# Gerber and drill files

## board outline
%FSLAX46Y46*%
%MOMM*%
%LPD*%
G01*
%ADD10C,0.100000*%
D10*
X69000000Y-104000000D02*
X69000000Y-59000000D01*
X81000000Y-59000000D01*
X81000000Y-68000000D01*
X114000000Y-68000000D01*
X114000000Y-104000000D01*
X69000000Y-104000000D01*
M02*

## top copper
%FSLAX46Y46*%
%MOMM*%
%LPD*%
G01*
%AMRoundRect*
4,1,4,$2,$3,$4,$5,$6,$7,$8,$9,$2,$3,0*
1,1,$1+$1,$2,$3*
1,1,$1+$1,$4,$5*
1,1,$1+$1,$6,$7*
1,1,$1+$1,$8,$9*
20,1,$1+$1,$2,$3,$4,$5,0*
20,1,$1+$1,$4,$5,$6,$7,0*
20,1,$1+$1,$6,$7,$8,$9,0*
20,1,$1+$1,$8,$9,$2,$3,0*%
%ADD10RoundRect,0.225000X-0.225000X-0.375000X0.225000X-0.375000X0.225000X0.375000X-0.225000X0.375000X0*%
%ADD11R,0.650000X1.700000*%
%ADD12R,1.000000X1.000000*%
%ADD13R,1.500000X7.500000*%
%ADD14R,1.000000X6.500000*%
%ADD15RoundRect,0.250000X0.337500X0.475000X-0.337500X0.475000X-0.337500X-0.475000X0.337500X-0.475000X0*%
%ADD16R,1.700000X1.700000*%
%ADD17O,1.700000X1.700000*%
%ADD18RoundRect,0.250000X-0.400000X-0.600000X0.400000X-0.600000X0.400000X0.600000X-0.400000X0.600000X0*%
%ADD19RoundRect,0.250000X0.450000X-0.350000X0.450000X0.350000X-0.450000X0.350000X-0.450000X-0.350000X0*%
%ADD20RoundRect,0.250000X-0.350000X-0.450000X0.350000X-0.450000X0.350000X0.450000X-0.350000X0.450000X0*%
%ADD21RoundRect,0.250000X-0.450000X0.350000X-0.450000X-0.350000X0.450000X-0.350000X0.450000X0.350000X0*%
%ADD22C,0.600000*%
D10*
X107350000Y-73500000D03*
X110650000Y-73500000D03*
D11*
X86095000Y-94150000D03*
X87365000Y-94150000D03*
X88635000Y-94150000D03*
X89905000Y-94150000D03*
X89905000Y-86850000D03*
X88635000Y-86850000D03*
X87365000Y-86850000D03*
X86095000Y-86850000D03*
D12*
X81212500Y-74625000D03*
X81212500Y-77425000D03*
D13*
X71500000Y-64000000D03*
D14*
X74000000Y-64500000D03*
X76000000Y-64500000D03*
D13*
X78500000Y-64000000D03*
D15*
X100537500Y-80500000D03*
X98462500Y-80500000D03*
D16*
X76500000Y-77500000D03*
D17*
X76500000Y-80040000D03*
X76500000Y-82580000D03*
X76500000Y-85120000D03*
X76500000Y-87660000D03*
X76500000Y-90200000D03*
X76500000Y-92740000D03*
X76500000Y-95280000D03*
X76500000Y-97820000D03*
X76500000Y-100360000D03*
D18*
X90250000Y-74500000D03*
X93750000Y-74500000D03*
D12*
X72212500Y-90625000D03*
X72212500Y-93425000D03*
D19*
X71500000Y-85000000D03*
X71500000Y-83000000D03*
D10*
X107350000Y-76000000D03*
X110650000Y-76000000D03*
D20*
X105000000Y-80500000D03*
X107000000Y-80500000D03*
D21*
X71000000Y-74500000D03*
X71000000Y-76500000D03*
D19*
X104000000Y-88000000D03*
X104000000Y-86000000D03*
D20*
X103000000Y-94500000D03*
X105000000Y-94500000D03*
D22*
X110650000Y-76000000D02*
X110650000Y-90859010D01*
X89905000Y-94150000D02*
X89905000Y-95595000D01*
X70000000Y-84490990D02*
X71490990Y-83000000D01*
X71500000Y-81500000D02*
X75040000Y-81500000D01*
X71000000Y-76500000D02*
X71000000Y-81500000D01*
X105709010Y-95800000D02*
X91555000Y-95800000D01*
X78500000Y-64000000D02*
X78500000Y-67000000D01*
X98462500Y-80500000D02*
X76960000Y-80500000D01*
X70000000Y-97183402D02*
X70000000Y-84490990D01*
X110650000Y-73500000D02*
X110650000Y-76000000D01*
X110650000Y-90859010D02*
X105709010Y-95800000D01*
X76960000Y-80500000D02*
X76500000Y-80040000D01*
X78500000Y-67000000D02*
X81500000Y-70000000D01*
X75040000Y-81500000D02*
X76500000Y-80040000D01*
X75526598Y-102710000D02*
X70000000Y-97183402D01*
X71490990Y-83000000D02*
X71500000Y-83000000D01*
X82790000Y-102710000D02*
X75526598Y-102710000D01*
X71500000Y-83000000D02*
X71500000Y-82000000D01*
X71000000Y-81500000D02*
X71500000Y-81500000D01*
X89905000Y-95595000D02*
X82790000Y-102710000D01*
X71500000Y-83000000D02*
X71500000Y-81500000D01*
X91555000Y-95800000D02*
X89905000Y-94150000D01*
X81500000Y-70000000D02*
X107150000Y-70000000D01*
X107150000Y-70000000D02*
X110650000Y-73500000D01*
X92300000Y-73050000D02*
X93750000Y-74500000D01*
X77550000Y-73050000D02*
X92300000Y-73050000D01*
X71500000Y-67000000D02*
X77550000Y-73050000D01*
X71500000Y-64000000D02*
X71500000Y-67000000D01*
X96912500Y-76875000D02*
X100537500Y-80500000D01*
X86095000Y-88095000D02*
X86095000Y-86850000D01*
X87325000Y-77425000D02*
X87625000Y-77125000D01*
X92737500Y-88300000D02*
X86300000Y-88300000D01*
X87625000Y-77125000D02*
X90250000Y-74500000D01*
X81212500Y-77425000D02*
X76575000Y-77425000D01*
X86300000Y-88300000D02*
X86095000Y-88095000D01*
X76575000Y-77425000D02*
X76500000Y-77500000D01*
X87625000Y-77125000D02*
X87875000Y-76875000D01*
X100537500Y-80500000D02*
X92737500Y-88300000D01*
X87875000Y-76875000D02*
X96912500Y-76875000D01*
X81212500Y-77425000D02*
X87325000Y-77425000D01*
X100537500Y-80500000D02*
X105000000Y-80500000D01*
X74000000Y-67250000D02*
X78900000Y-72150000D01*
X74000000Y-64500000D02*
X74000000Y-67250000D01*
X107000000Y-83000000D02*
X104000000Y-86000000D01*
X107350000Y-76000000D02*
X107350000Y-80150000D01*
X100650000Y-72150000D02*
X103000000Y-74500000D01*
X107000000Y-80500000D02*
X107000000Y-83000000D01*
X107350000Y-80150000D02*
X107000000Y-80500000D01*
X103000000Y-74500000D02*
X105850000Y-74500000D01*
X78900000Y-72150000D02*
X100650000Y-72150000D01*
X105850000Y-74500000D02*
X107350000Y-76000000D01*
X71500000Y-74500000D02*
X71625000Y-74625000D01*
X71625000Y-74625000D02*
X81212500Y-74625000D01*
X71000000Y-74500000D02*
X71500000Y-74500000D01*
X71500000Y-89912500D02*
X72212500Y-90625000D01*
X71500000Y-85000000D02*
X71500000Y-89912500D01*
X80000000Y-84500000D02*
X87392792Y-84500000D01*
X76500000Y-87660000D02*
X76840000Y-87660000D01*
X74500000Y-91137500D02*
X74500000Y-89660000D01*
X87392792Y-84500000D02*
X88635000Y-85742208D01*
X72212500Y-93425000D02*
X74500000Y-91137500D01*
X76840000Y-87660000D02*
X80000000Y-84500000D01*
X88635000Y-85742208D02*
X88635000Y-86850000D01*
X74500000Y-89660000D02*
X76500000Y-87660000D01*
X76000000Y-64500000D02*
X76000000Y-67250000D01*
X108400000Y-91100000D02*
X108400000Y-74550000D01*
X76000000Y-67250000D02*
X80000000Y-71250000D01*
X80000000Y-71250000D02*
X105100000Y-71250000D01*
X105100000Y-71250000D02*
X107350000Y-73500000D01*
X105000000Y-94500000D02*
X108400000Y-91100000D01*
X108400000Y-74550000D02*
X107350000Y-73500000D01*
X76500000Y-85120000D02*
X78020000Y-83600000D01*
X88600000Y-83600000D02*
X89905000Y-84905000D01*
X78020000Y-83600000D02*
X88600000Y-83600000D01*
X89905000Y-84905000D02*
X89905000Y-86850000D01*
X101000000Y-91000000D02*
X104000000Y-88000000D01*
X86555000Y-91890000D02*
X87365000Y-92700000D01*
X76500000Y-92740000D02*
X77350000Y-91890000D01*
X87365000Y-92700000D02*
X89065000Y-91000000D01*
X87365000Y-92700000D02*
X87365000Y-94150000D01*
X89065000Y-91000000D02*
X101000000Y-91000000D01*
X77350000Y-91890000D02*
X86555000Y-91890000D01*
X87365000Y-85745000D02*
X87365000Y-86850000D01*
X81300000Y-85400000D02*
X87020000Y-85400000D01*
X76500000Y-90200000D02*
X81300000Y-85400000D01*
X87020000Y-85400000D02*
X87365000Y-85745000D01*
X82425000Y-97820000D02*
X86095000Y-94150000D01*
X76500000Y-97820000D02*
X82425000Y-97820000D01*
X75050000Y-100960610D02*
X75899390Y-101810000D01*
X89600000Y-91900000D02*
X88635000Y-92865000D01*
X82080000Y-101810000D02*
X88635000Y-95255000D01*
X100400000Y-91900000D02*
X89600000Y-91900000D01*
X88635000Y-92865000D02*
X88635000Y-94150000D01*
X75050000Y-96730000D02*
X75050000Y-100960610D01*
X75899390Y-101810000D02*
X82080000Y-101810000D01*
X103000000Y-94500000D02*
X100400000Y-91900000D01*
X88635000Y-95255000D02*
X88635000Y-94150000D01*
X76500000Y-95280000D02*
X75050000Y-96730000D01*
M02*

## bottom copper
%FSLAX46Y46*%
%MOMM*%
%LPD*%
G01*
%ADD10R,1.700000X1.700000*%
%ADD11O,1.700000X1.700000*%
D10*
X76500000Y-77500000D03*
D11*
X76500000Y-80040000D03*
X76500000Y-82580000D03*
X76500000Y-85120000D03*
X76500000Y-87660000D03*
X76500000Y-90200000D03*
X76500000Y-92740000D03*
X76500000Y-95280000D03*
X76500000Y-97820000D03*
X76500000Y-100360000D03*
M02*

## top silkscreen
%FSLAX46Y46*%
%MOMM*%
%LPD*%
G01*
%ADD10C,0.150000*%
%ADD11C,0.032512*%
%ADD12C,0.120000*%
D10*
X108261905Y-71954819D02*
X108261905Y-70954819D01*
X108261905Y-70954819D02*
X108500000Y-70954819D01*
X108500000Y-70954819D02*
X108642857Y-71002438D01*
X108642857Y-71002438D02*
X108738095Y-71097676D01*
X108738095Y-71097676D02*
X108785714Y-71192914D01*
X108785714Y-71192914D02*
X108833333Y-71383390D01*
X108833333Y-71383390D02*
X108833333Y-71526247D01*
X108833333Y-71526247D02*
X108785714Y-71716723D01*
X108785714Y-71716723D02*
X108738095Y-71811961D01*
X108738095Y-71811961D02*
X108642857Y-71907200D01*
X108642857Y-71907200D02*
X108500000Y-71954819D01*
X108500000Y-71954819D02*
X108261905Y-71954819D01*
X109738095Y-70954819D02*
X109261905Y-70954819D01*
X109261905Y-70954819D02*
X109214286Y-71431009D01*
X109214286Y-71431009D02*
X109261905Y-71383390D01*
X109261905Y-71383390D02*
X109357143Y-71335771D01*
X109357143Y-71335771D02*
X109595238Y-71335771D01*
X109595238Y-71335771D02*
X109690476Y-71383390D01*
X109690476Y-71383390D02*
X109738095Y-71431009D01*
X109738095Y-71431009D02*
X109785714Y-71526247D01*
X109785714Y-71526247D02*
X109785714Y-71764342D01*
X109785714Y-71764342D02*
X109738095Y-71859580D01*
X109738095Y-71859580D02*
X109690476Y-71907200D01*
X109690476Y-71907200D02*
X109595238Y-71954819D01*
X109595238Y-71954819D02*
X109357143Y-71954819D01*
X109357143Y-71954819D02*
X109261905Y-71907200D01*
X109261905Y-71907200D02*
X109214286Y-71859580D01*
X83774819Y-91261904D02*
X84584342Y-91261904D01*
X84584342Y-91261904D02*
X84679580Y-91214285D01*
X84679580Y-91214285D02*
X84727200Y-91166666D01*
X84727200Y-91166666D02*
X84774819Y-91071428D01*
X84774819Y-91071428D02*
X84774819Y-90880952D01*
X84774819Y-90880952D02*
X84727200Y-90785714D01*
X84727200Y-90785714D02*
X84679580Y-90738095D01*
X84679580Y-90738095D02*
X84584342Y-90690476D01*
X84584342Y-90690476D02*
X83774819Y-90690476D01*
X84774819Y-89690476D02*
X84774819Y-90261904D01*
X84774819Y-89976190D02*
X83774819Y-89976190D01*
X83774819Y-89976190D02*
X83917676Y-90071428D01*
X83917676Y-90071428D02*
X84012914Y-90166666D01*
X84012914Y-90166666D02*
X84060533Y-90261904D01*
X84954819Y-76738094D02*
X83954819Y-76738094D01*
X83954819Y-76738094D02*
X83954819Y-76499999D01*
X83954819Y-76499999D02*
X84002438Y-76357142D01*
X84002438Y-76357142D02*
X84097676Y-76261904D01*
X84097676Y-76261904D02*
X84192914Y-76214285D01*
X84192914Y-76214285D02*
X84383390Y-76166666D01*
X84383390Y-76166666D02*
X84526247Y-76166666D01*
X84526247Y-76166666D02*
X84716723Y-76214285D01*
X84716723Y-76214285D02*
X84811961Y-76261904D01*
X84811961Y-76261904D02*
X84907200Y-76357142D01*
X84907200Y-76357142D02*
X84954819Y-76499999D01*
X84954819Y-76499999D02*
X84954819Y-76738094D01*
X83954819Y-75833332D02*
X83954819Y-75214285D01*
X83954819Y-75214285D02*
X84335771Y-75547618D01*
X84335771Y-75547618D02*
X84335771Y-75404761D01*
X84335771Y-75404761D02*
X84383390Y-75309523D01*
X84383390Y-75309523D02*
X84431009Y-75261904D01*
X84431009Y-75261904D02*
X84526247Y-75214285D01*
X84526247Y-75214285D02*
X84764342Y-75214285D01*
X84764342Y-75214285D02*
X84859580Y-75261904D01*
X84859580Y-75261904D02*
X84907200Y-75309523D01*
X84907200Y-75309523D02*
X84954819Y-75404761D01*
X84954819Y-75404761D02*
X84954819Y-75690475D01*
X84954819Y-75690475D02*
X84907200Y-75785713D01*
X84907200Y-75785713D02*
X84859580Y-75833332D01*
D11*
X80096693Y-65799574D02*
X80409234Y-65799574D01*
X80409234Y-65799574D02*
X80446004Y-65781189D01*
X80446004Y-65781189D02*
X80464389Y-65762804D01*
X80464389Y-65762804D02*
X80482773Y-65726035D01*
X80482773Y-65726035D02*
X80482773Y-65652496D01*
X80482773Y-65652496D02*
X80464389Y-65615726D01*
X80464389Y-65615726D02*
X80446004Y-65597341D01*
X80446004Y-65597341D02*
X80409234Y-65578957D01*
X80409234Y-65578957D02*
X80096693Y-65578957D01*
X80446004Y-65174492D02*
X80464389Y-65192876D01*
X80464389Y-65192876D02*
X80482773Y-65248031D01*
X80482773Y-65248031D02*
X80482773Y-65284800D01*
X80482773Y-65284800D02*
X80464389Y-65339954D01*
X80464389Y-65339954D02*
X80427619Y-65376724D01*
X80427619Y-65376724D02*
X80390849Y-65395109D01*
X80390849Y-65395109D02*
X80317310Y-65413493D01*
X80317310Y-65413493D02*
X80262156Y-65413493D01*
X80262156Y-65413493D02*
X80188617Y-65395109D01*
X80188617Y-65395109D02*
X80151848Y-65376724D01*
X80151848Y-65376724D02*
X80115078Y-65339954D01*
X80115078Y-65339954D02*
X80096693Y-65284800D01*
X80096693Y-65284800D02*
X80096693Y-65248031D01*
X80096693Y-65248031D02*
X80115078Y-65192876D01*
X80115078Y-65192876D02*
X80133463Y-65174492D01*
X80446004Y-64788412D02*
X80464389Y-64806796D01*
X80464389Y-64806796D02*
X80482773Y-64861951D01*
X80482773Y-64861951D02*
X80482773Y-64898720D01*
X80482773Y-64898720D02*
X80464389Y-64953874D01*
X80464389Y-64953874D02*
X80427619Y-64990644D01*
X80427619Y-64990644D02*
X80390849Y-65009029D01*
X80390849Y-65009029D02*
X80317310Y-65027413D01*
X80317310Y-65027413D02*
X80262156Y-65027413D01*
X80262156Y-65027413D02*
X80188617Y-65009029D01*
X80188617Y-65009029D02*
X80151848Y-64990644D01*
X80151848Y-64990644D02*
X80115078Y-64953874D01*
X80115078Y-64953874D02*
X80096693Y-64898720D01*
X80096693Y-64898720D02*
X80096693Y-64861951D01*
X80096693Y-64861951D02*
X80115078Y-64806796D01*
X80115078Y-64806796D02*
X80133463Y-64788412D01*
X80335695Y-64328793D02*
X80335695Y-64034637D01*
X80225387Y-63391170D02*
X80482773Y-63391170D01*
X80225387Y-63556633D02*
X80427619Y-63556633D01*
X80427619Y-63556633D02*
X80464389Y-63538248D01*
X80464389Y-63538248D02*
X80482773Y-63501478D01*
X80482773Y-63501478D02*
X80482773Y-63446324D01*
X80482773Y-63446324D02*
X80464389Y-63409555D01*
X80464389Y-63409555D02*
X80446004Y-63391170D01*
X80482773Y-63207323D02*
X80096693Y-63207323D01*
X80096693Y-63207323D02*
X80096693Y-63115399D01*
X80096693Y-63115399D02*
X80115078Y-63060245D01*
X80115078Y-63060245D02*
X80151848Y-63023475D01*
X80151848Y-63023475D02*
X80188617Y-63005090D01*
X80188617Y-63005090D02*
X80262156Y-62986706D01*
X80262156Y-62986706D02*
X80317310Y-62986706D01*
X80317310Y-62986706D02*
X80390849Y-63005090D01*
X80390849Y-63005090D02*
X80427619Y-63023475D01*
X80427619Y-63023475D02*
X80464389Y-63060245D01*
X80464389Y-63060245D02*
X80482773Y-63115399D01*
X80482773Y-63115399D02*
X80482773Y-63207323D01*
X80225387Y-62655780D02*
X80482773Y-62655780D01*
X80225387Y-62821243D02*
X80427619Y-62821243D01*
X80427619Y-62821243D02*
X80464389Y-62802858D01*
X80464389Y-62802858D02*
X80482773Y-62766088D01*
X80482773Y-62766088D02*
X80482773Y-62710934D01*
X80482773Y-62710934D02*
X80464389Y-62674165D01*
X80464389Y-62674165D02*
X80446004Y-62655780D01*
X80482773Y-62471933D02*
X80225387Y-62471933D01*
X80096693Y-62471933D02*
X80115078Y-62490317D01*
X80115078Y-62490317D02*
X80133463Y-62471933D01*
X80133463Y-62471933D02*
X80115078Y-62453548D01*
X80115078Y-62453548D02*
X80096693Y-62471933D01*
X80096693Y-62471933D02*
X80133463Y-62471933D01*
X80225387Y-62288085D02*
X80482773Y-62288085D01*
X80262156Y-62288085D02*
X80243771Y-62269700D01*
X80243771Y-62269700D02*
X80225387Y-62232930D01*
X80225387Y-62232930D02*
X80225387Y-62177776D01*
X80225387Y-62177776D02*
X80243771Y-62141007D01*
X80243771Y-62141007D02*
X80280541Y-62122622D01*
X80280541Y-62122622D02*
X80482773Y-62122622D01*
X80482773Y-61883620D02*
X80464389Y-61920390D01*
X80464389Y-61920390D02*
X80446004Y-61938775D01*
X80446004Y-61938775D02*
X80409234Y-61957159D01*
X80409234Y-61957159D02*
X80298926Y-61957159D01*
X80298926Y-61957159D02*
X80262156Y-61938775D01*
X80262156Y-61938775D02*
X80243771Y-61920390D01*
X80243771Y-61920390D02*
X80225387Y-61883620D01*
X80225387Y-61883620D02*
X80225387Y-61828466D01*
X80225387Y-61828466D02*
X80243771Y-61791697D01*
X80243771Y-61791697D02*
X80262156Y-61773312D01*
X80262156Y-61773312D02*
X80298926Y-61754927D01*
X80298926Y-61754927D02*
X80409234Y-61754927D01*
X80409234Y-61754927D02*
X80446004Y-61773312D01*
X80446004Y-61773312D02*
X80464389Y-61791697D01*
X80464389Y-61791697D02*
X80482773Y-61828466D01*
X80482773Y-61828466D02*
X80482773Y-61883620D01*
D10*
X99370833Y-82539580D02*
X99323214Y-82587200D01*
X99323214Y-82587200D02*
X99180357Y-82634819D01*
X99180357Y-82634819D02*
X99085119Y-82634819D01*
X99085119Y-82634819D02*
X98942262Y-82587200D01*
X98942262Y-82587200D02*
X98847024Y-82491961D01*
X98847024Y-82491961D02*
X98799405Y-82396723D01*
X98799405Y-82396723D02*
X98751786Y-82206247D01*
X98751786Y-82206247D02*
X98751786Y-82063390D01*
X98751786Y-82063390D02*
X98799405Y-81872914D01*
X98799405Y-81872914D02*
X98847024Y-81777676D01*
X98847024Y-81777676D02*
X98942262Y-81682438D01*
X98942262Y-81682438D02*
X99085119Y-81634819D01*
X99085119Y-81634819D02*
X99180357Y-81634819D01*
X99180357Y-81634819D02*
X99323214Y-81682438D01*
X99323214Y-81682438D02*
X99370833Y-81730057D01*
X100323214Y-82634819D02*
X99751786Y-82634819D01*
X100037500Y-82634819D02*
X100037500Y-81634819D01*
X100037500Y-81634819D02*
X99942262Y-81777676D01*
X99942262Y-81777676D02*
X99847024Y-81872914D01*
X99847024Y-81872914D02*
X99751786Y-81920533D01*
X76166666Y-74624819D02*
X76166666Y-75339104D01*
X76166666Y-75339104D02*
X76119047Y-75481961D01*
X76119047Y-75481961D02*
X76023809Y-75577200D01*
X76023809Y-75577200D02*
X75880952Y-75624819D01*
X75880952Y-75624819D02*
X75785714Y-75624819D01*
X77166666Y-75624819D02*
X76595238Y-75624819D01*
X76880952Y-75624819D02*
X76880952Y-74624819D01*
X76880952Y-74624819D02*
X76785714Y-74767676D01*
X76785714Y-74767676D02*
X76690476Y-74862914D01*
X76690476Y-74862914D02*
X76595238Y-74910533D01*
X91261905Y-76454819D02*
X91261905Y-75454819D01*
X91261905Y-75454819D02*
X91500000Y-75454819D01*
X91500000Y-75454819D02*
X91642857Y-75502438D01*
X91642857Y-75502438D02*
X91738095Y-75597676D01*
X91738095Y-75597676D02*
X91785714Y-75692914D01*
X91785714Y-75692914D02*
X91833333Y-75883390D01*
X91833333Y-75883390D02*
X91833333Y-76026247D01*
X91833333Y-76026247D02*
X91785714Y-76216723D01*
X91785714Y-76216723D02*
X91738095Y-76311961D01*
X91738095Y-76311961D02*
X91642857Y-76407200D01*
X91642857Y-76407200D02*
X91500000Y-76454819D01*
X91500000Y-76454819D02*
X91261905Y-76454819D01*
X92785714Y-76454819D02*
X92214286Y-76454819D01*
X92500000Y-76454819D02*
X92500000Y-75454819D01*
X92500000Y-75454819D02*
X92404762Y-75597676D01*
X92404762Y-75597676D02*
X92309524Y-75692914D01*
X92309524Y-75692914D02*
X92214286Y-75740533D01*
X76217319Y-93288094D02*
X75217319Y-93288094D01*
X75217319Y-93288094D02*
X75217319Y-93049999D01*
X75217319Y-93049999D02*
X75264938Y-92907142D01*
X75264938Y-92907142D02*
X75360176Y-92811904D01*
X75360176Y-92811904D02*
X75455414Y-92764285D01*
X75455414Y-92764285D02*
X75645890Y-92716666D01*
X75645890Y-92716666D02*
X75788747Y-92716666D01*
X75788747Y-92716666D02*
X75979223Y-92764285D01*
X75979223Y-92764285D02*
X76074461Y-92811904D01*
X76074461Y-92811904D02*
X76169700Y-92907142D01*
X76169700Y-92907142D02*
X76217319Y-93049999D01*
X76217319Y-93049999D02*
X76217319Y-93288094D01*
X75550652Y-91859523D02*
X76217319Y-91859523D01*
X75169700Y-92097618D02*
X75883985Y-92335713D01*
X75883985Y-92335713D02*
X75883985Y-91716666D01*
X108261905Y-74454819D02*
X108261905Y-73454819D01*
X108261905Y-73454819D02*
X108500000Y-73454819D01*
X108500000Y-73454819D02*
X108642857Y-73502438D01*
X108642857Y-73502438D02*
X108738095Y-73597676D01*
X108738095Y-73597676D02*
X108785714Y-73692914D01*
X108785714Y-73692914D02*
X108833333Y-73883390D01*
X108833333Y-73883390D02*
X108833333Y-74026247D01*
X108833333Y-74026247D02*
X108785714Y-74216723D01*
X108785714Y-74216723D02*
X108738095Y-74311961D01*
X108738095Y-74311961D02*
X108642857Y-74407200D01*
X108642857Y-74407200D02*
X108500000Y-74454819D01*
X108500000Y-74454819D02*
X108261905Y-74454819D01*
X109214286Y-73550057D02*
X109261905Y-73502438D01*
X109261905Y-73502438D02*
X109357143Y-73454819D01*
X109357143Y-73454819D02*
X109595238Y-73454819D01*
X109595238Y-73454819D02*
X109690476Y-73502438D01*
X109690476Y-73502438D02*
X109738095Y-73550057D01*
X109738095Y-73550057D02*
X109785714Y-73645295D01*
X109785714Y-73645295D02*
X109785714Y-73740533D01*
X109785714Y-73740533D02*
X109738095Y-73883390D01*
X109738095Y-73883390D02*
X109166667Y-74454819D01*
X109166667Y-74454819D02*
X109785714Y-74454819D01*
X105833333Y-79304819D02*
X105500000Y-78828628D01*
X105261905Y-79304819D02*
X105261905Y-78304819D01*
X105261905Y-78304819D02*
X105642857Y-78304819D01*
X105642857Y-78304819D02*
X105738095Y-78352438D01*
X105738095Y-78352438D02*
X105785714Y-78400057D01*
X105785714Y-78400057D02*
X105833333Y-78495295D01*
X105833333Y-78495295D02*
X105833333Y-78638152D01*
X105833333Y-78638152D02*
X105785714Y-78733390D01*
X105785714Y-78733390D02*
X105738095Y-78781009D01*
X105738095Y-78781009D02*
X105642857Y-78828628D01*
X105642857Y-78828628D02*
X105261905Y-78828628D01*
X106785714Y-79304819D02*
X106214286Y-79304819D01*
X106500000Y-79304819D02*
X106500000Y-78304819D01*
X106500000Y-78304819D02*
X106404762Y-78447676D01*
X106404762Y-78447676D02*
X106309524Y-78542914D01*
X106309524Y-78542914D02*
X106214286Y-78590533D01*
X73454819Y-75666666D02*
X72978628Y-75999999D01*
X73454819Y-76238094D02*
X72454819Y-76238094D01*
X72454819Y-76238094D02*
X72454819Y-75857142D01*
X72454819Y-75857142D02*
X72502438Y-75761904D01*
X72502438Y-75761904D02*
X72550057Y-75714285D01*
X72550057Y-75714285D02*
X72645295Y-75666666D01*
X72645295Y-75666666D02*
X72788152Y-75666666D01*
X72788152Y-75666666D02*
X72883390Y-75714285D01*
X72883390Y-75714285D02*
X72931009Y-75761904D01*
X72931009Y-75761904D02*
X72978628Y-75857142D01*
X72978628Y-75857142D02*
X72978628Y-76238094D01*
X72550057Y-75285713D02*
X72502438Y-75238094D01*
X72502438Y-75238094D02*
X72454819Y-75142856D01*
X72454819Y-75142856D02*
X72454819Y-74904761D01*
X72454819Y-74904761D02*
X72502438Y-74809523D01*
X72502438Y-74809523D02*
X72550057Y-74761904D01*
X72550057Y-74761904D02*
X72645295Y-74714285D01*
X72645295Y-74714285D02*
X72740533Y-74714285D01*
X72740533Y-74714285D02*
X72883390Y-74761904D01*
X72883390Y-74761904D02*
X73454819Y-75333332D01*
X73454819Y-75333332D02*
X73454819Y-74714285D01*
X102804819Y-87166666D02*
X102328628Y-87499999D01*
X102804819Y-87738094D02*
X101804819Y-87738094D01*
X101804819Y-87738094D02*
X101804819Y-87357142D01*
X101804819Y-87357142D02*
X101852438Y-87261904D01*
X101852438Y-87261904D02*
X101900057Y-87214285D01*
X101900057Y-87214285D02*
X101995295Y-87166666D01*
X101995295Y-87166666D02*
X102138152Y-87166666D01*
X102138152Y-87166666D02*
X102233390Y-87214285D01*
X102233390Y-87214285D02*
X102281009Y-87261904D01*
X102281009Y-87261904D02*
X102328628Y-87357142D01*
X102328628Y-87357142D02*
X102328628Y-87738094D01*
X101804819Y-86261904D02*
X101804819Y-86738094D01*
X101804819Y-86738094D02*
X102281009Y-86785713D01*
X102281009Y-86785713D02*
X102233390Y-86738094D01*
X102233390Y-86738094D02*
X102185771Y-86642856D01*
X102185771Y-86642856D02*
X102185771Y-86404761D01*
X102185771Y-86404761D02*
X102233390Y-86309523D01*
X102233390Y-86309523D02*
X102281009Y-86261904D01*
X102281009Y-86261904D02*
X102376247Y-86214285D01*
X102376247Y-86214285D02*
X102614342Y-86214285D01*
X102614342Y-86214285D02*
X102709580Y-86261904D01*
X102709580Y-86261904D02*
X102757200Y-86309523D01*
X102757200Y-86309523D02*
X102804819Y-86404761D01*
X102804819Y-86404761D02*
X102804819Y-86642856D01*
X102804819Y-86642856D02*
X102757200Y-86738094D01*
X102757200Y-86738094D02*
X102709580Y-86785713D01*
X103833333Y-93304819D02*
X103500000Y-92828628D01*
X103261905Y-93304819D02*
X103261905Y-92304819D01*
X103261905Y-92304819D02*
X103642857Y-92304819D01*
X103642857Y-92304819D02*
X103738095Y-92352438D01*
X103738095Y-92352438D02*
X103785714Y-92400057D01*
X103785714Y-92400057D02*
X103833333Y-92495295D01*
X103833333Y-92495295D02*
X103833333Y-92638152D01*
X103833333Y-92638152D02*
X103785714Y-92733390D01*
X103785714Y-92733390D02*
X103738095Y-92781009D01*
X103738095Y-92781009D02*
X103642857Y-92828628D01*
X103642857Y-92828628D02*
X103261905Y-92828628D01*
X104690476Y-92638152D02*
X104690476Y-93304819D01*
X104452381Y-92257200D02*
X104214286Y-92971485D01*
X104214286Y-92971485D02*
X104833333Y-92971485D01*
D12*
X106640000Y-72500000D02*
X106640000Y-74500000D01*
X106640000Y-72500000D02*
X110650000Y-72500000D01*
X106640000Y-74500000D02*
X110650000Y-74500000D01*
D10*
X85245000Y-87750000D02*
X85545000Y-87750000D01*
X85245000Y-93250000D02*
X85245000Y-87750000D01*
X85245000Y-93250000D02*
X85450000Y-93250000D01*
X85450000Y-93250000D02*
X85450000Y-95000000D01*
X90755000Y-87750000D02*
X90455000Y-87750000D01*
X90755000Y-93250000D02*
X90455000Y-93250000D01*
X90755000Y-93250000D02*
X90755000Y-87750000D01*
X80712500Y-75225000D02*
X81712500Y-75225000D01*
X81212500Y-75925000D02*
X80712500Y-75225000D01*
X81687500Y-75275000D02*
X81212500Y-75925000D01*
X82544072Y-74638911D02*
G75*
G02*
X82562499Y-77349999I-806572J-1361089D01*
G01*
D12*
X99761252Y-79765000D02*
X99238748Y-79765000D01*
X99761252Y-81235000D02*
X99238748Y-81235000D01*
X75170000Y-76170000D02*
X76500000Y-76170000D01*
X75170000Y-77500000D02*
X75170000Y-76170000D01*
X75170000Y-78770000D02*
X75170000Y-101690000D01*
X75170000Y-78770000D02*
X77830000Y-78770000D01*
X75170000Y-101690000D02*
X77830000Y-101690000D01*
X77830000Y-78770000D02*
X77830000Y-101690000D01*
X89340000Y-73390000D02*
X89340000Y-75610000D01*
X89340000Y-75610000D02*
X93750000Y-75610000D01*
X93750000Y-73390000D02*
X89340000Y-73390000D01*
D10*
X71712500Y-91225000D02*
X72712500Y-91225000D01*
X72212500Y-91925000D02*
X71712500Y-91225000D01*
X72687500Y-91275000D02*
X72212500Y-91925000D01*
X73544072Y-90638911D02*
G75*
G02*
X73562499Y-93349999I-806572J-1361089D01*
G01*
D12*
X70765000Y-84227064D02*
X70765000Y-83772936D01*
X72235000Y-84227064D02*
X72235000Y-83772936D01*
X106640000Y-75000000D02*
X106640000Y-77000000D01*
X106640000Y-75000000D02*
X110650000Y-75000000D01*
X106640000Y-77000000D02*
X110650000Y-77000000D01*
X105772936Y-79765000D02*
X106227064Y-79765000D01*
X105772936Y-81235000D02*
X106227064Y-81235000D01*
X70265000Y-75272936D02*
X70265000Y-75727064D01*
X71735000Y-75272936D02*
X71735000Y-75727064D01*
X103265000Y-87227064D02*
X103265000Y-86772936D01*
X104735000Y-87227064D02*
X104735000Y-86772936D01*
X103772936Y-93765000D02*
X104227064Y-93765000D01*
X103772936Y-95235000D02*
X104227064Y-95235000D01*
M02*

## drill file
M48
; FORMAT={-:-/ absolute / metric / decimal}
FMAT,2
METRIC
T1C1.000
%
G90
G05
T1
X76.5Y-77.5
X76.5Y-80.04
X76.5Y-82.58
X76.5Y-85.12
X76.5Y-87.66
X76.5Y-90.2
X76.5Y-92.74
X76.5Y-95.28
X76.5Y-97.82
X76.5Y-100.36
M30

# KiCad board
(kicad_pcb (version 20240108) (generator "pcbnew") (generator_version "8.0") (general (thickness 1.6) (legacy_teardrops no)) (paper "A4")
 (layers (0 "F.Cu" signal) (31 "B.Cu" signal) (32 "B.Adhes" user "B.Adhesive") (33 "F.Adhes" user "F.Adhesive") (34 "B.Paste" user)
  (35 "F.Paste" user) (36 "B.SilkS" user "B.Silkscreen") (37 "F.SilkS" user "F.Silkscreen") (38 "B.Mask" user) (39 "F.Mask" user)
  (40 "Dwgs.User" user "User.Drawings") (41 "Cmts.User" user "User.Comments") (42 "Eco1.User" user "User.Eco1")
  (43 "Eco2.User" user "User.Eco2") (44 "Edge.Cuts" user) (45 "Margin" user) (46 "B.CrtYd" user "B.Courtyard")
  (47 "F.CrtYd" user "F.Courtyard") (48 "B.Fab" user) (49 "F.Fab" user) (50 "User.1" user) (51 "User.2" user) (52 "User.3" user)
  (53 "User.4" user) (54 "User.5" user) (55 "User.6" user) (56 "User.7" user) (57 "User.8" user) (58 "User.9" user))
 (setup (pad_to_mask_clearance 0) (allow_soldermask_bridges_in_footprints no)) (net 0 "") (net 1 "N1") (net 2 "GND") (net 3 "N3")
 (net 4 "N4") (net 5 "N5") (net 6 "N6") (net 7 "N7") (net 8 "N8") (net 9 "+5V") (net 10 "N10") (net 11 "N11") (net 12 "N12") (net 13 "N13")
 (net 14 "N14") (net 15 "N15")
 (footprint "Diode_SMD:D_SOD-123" (layer "F.Cu") (at 109 73.5)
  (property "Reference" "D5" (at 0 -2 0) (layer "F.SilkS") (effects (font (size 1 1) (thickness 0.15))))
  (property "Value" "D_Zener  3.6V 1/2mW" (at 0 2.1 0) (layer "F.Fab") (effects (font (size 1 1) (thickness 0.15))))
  (fp_line (start -2.36 -1) (end -2.36 1) (stroke (width 0.12) (type solid)) (layer "F.SilkS"))
  (fp_line (start -2.36 -1) (end 1.65 -1) (stroke (width 0.12) (type solid)) (layer "F.SilkS"))
  (fp_line (start -2.36 1) (end 1.65 1) (stroke (width 0.12) (type solid)) (layer "F.SilkS"))
  (pad "1" smd roundrect (at -1.65 0) (size 0.9 1.2) (layers "F.Cu" "F.Paste" "F.Mask") (roundrect_rratio 0.25) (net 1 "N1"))
  (pad "2" smd roundrect (at 1.65 0) (size 0.9 1.2) (layers "F.Cu" "F.Paste" "F.Mask") (roundrect_rratio 0.25) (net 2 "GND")))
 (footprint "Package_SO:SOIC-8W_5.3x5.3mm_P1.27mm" (layer "F.Cu") (at 88 90.5 90)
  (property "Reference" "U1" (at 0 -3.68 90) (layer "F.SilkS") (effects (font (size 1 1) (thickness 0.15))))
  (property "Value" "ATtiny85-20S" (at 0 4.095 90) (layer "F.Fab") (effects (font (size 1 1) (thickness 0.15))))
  (fp_line (start 2.75 -2.755) (end 2.75 -2.455) (stroke (width 0.15) (type solid)) (layer "F.SilkS"))
  (fp_line (start -2.75 -2.755) (end 2.75 -2.755) (stroke (width 0.15) (type solid)) (layer "F.SilkS"))
  (fp_line (start -2.75 -2.755) (end -2.75 -2.55) (stroke (width 0.15) (type solid)) (layer "F.SilkS"))
  (fp_line (start -2.75 -2.55) (end -4.5 -2.55) (stroke (width 0.15) (type solid)) (layer "F.SilkS"))
  (fp_line (start 2.75 2.755) (end 2.75 2.455) (stroke (width 0.15) (type solid)) (layer "F.SilkS"))
  (fp_line (start -2.75 2.755) (end -2.75 2.455) (stroke (width 0.15) (type solid)) (layer "F.SilkS"))
  (fp_line (start -2.75 2.755) (end 2.75 2.755) (stroke (width 0.15) (type solid)) (layer "F.SilkS"))
  (pad "1" smd rect (at -3.65 -1.905 90) (size 1.7 0.65) (layers "F.Cu" "F.Paste" "F.Mask") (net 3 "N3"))
  (pad "2" smd rect (at -3.65 -0.635 90) (size 1.7 0.65) (layers "F.Cu" "F.Paste" "F.Mask") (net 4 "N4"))
  (pad "3" smd rect (at -3.65 0.635 90) (size 1.7 0.65) (layers "F.Cu" "F.Paste" "F.Mask") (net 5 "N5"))
  (pad "4" smd rect (at -3.65 1.905 90) (size 1.7 0.65) (layers "F.Cu" "F.Paste" "F.Mask") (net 2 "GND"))
  (pad "5" smd rect (at 3.65 1.905 90) (size 1.7 0.65) (layers "F.Cu" "F.Paste" "F.Mask") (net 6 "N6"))
  (pad "6" smd rect (at 3.65 0.635 90) (size 1.7 0.65) (layers "F.Cu" "F.Paste" "F.Mask") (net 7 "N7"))
  (pad "7" smd rect (at 3.65 -0.635 90) (size 1.7 0.65) (layers "F.Cu" "F.Paste" "F.Mask") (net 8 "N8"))
  (pad "8" smd rect (at 3.65 -1.905 90) (size 1.7 0.65) (layers "F.Cu" "F.Paste" "F.Mask") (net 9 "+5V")))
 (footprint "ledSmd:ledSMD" (layer "F.Cu") (at 81.2125 76.425 -90)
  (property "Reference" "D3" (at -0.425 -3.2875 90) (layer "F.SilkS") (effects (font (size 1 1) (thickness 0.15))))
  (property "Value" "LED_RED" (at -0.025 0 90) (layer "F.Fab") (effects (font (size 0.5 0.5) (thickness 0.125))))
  (fp_line (start -1.2 0.5) (end -1.2 -0.5) (stroke (width 0.15) (type solid)) (layer "F.SilkS"))
  (fp_line (start -0.5 0) (end -1.2 0.5) (stroke (width 0.15) (type solid)) (layer "F.SilkS"))
  (fp_line (start -1.15 -0.475) (end -0.5 0) (stroke (width 0.15) (type solid)) (layer "F.SilkS"))
  (fp_arc (start -1.786089 -1.331572) (mid -0.435753 -2.107089) (end 0.924999 -1.349999) (stroke (width 0.15) (type solid))
   (layer "F.SilkS"))
  (pad "1" smd rect (at -1.8 0 270) (size 1 1) (layers "F.Cu" "F.Paste" "F.Mask") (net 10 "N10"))
  (pad "2" smd rect (at 1 0 270) (size 1 1) (layers "F.Cu" "F.Paste" "F.Mask") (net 9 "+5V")))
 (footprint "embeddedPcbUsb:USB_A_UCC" (layer "F.Cu") (at 75 64.2 -90)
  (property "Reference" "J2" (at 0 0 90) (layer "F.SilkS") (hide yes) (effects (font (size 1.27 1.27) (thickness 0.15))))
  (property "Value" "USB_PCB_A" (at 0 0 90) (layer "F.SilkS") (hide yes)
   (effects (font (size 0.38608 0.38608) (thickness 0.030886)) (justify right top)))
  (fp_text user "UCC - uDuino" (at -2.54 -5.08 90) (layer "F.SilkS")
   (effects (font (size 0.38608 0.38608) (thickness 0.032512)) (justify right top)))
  (pad "1" smd rect (at -0.2 3.5 270) (size 7.5 1.5) (layers "F.Cu" "F.Paste" "F.Mask") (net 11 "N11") (solder_mask_margin 0.1016))
  (pad "2" smd rect (at 0.3 1 270) (size 6.5 1) (layers "F.Cu" "F.Paste" "F.Mask") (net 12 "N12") (solder_mask_margin 0.1016))
  (pad "3" smd rect (at 0.3 -1 270) (size 6.5 1) (layers "F.Cu" "F.Paste" "F.Mask") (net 1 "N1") (solder_mask_margin 0.1016))
  (pad "4" smd rect (at -0.2 -3.5 270) (size 7.5 1.5) (layers "F.Cu" "F.Paste" "F.Mask") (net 2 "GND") (solder_mask_margin 0.1016)))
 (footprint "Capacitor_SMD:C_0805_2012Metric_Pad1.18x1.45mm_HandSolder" (layer "F.Cu") (at 99.5 80.5 180)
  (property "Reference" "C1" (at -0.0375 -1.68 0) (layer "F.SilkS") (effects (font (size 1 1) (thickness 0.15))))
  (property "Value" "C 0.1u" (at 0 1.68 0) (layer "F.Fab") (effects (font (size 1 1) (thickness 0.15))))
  (fp_line (start -0.261252 0.735) (end 0.261252 0.735) (stroke (width 0.12) (type solid)) (layer "F.SilkS"))
  (fp_line (start -0.261252 -0.735) (end 0.261252 -0.735) (stroke (width 0.12) (type solid)) (layer "F.SilkS"))
  (pad "1" smd roundrect (at -1.0375 0 180) (size 1.175 1.45) (layers "F.Cu" "F.Paste" "F.Mask") (roundrect_rratio 0.212766) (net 9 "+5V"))
  (pad "2" smd roundrect (at 1.0375 0 180) (size 1.175 1.45) (layers "F.Cu" "F.Paste" "F.Mask") (roundrect_rratio 0.212766) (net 2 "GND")))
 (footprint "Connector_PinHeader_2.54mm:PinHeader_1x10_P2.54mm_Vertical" (layer "F.Cu") (at 76.5 77.5)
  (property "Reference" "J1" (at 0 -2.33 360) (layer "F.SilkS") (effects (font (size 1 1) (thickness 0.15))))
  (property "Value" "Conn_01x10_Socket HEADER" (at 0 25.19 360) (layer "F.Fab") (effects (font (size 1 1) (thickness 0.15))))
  (fp_line (start -1.33 -1.33) (end 0 -1.33) (stroke (width 0.12) (type solid)) (layer "F.SilkS"))
  (fp_line (start -1.33 0) (end -1.33 -1.33) (stroke (width 0.12) (type solid)) (layer "F.SilkS"))
  (fp_line (start -1.33 1.27) (end -1.33 24.19) (stroke (width 0.12) (type solid)) (layer "F.SilkS"))
  (fp_line (start -1.33 1.27) (end 1.33 1.27) (stroke (width 0.12) (type solid)) (layer "F.SilkS"))
  (fp_line (start -1.33 24.19) (end 1.33 24.19) (stroke (width 0.12) (type solid)) (layer "F.SilkS"))
  (fp_line (start 1.33 1.27) (end 1.33 24.19) (stroke (width 0.12) (type solid)) (layer "F.SilkS"))
  (pad "1" thru_hole rect (at 0 0) (size 1.7 1.7) (drill 1) (layers "*.Cu" "*.Mask") (remove_unused_layers no) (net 9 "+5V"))
  (pad "2" thru_hole oval (at 0 2.54) (size 1.7 1.7) (drill 1) (layers "*.Cu" "*.Mask") (remove_unused_layers no) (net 2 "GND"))
  (pad "3" thru_hole oval (at 0 5.08) (size 1.7 1.7) (drill 1) (layers "*.Cu" "*.Mask") (remove_unused_layers no) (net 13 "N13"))
  (pad "4" thru_hole oval (at 0 7.62) (size 1.7 1.7) (drill 1) (layers "*.Cu" "*.Mask") (remove_unused_layers no) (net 6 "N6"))
  (pad "5" thru_hole oval (at 0 10.16) (size 1.7 1.7) (drill 1) (layers "*.Cu" "*.Mask") (remove_unused_layers no) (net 7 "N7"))
  (pad "6" thru_hole oval (at 0 12.7) (size 1.7 1.7) (drill 1) (layers "*.Cu" "*.Mask") (remove_unused_layers no) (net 8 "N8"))
  (pad "7" thru_hole oval (at 0 15.24) (size 1.7 1.7) (drill 1) (layers "*.Cu" "*.Mask") (remove_unused_layers no) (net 4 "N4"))
  (pad "8" thru_hole oval (at 0 17.78) (size 1.7 1.7) (drill 1) (layers "*.Cu" "*.Mask") (remove_unused_layers no) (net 5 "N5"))
  (pad "9" thru_hole oval (at 0 20.32) (size 1.7 1.7) (drill 1) (layers "*.Cu" "*.Mask") (remove_unused_layers no) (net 3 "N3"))
  (pad "10" thru_hole oval (at 0 22.86) (size 1.7 1.7) (drill 1) (layers "*.Cu" "*.Mask") (remove_unused_layers no) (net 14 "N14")))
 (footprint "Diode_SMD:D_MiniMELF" (layer "F.Cu") (at 92 74.5)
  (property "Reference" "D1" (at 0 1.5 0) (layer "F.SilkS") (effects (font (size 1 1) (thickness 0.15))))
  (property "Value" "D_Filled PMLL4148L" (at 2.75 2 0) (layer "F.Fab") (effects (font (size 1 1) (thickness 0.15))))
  (fp_line (start -2.66 -1.11) (end -2.66 1.11) (stroke (width 0.12) (type solid)) (layer "F.SilkS"))
  (fp_line (start -2.66 1.11) (end 1.75 1.11) (stroke (width 0.12) (type solid)) (layer "F.SilkS"))
  (fp_line (start 1.75 -1.11) (end -2.66 -1.11) (stroke (width 0.12) (type solid)) (layer "F.SilkS"))
  (pad "1" smd roundrect (at -1.75 0) (size 1.3 1.7) (layers "F.Cu" "F.Paste" "F.Mask") (roundrect_rratio 0.1923076923) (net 9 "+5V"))
  (pad "2" smd roundrect (at 1.75 0) (size 1.3 1.7) (layers "F.Cu" "F.Paste" "F.Mask") (roundrect_rratio 0.1923076923) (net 11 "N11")))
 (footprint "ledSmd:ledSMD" (layer "F.Cu") (at 72.2125 92.425 -90)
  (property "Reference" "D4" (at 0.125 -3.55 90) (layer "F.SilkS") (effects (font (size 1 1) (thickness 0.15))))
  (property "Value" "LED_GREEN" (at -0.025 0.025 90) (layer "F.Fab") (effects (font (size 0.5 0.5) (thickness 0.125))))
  (fp_line (start -1.2 0.5) (end -1.2 -0.5) (stroke (width 0.15) (type solid)) (layer "F.SilkS"))
  (fp_line (start -0.5 0) (end -1.2 0.5) (stroke (width 0.15) (type solid)) (layer "F.SilkS"))
  (fp_line (start -1.15 -0.475) (end -0.5 0) (stroke (width 0.15) (type solid)) (layer "F.SilkS"))
  (fp_arc (start -1.786089 -1.331572) (mid -0.435753 -2.107089) (end 0.924999 -1.349999) (stroke (width 0.15) (type solid))
   (layer "F.SilkS"))
  (pad "1" smd rect (at -1.8 0 270) (size 1 1) (layers "F.Cu" "F.Paste" "F.Mask") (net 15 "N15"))
  (pad "2" smd rect (at 1 0 270) (size 1 1) (layers "F.Cu" "F.Paste" "F.Mask") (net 7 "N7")))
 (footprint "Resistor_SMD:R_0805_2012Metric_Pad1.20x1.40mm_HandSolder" (layer "F.Cu") (at 71.5 84 90)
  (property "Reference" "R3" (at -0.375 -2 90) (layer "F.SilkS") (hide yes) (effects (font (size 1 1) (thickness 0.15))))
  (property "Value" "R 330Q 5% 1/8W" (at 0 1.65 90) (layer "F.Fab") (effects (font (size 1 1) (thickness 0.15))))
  (fp_line (start -0.227064 -0.735) (end 0.227064 -0.735) (stroke (width 0.12) (type solid)) (layer "F.SilkS"))
  (fp_line (start -0.227064 0.735) (end 0.227064 0.735) (stroke (width 0.12) (type solid)) (layer "F.SilkS"))
  (pad "1" smd roundrect (at -1 0 90) (size 1.2 1.4) (layers "F.Cu" "F.Paste" "F.Mask") (roundrect_rratio 0.208333) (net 15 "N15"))
  (pad "2" smd roundrect (at 1 0 90) (size 1.2 1.4) (layers "F.Cu" "F.Paste" "F.Mask") (roundrect_rratio 0.208333) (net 2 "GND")))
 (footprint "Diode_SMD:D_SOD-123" (layer "F.Cu") (at 109 76)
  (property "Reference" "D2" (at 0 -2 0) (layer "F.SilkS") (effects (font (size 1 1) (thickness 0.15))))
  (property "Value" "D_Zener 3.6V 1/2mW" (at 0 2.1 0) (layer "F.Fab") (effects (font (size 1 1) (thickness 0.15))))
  (fp_line (start -2.36 -1) (end -2.36 1) (stroke (width 0.12) (type solid)) (layer "F.SilkS"))
  (fp_line (start -2.36 -1) (end 1.65 -1) (stroke (width 0.12) (type solid)) (layer "F.SilkS"))
  (fp_line (start -2.36 1) (end 1.65 1) (stroke (width 0.12) (type solid)) (layer "F.SilkS"))
  (pad "1" smd roundrect (at -1.65 0) (size 0.9 1.2) (layers "F.Cu" "F.Paste" "F.Mask") (roundrect_rratio 0.25) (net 12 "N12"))
  (pad "2" smd roundrect (at 1.65 0) (size 0.9 1.2) (layers "F.Cu" "F.Paste" "F.Mask") (roundrect_rratio 0.25) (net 2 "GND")))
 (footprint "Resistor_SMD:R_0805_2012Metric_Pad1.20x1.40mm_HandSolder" (layer "F.Cu") (at 106 80.5)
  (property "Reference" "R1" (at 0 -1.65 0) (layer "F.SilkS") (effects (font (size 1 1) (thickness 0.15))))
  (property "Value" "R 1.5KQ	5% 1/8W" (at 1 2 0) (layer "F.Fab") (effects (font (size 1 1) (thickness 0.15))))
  (fp_line (start -0.227064 -0.735) (end 0.227064 -0.735) (stroke (width 0.12) (type solid)) (layer "F.SilkS"))
  (fp_line (start -0.227064 0.735) (end 0.227064 0.735) (stroke (width 0.12) (type solid)) (layer "F.SilkS"))
  (pad "1" smd roundrect (at -1 0) (size 1.2 1.4) (layers "F.Cu" "F.Paste" "F.Mask") (roundrect_rratio 0.208333) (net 9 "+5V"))
  (pad "2" smd roundrect (at 1 0) (size 1.2 1.4) (layers "F.Cu" "F.Paste" "F.Mask") (roundrect_rratio 0.208333) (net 12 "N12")))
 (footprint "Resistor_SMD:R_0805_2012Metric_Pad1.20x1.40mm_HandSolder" (layer "F.Cu") (at 71 75.5 -90)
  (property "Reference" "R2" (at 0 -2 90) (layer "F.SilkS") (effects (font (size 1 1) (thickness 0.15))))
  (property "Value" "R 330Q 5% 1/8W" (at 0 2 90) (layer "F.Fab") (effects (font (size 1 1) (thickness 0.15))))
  (fp_line (start -0.227064 0.735) (end 0.227064 0.735) (stroke (width 0.12) (type solid)) (layer "F.SilkS"))
  (fp_line (start -0.227064 -0.735) (end 0.227064 -0.735) (stroke (width 0.12) (type solid)) (layer "F.SilkS"))
  (pad "1" smd roundrect (at -1 0 270) (size 1.2 1.4) (layers "F.Cu" "F.Paste" "F.Mask") (roundrect_rratio 0.208333) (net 10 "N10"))
  (pad "2" smd roundrect (at 1 0 270) (size 1.2 1.4) (layers "F.Cu" "F.Paste" "F.Mask") (roundrect_rratio 0.208333) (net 2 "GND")))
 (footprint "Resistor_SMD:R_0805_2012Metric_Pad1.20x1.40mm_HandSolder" (layer "F.Cu") (at 104 87 90)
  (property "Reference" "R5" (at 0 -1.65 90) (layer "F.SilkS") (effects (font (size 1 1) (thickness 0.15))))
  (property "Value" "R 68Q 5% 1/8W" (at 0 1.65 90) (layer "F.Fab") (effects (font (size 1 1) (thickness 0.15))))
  (fp_line (start -0.227064 -0.735) (end 0.227064 -0.735) (stroke (width 0.12) (type solid)) (layer "F.SilkS"))
  (fp_line (start -0.227064 0.735) (end 0.227064 0.735) (stroke (width 0.12) (type solid)) (layer "F.SilkS"))
  (pad "1" smd roundrect (at -1 0 90) (size 1.2 1.4) (layers "F.Cu" "F.Paste" "F.Mask") (roundrect_rratio 0.208333) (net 4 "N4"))
  (pad "2" smd roundrect (at 1 0 90) (size 1.2 1.4) (layers "F.Cu" "F.Paste" "F.Mask") (roundrect_rratio 0.208333) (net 12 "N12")))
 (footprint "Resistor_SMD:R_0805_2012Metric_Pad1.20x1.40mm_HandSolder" (layer "F.Cu") (at 104 94.5)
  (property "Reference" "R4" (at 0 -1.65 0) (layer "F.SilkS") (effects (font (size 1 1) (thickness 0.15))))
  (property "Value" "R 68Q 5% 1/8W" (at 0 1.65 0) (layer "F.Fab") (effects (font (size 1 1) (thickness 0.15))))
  (fp_line (start -0.227064 -0.735) (end 0.227064 -0.735) (stroke (width 0.12) (type solid)) (layer "F.SilkS"))
  (fp_line (start -0.227064 0.735) (end 0.227064 0.735) (stroke (width 0.12) (type solid)) (layer "F.SilkS"))
  (pad "1" smd roundrect (at -1 0) (size 1.2 1.4) (layers "F.Cu" "F.Paste" "F.Mask") (roundrect_rratio 0.208333) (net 5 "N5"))
  (pad "2" smd roundrect (at 1 0) (size 1.2 1.4) (layers "F.Cu" "F.Paste" "F.Mask") (roundrect_rratio 0.208333) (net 1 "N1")))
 (gr_poly
  (pts (xy 69 104) (xy 69 59) (xy 81 59) (xy 81 68) (xy 114 68) (xy 114 104)) (stroke (width 0.1) (type solid)) (fill none)
  (layer "Edge.Cuts"))
 (segment (start 110.65 76) (end 110.65 90.85901) (width 0.6) (layer "F.Cu") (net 2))
 (segment (start 89.905 94.15) (end 89.905 95.595) (width 0.6) (layer "F.Cu") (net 2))
 (segment (start 70 84.49099) (end 71.49099 83) (width 0.6) (layer "F.Cu") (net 2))
 (segment (start 71.5 81.5) (end 75.04 81.5) (width 0.6) (layer "F.Cu") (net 2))
 (segment (start 71 76.5) (end 71 81.5) (width 0.6) (layer "F.Cu") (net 2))
 (segment (start 105.70901 95.8) (end 91.555 95.8) (width 0.6) (layer "F.Cu") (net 2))
 (segment (start 78.5 64) (end 78.5 67) (width 0.6) (layer "F.Cu") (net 2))
 (segment (start 98.4625 80.5) (end 76.96 80.5) (width 0.6) (layer "F.Cu") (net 2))
 (segment (start 70 97.183402) (end 70 84.49099) (width 0.6) (layer "F.Cu") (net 2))
 (segment (start 110.65 73.5) (end 110.65 76) (width 0.6) (layer "F.Cu") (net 2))
 (segment (start 110.65 90.85901) (end 105.70901 95.8) (width 0.6) (layer "F.Cu") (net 2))
 (segment (start 76.96 80.5) (end 76.5 80.04) (width 0.6) (layer "F.Cu") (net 2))
 (segment (start 78.5 67) (end 81.5 70) (width 0.6) (layer "F.Cu") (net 2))
 (segment (start 75.04 81.5) (end 76.5 80.04) (width 0.6) (layer "F.Cu") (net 2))
 (segment (start 75.526598 102.71) (end 70 97.183402) (width 0.6) (layer "F.Cu") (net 2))
 (segment (start 71.49099 83) (end 71.5 83) (width 0.6) (layer "F.Cu") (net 2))
 (segment (start 82.79 102.71) (end 75.526598 102.71) (width 0.6) (layer "F.Cu") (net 2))
 (segment (start 71.5 83) (end 71.5 82) (width 0.6) (layer "F.Cu") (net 2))
 (segment (start 71 81.5) (end 71.5 81.5) (width 0.6) (layer "F.Cu") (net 2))
 (segment (start 89.905 95.595) (end 82.79 102.71) (width 0.6) (layer "F.Cu") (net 2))
 (segment (start 71.5 83) (end 71.5 81.5) (width 0.6) (layer "F.Cu") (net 2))
 (segment (start 91.555 95.8) (end 89.905 94.15) (width 0.6) (layer "F.Cu") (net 2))
 (segment (start 81.5 70) (end 107.15 70) (width 0.6) (layer "F.Cu") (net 2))
 (segment (start 107.15 70) (end 110.65 73.5) (width 0.6) (layer "F.Cu") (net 2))
 (segment (start 92.3 73.05) (end 93.75 74.5) (width 0.6) (layer "F.Cu") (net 11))
 (segment (start 77.55 73.05) (end 92.3 73.05) (width 0.6) (layer "F.Cu") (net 11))
 (segment (start 71.5 67) (end 77.55 73.05) (width 0.6) (layer "F.Cu") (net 11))
 (segment (start 71.5 64) (end 71.5 67) (width 0.6) (layer "F.Cu") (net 11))
 (segment (start 96.9125 76.875) (end 100.5375 80.5) (width 0.6) (layer "F.Cu") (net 9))
 (segment (start 86.095 88.095) (end 86.095 86.85) (width 0.6) (layer "F.Cu") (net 9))
 (segment (start 87.325 77.425) (end 87.625 77.125) (width 0.6) (layer "F.Cu") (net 9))
 (segment (start 92.7375 88.3) (end 86.3 88.3) (width 0.6) (layer "F.Cu") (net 9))
 (segment (start 87.625 77.125) (end 90.25 74.5) (width 0.6) (layer "F.Cu") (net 9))
 (segment (start 81.2125 77.425) (end 76.575 77.425) (width 0.6) (layer "F.Cu") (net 9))
 (segment (start 86.3 88.3) (end 86.095 88.095) (width 0.6) (layer "F.Cu") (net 9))
 (segment (start 76.575 77.425) (end 76.5 77.5) (width 0.6) (layer "F.Cu") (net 9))
 (segment (start 87.625 77.125) (end 87.875 76.875) (width 0.6) (layer "F.Cu") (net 9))
 (segment (start 100.5375 80.5) (end 92.7375 88.3) (width 0.6) (layer "F.Cu") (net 9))
 (segment (start 87.875 76.875) (end 96.9125 76.875) (width 0.6) (layer "F.Cu") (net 9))
 (segment (start 81.2125 77.425) (end 87.325 77.425) (width 0.6) (layer "F.Cu") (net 9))
 (segment (start 100.5375 80.5) (end 105 80.5) (width 0.6) (layer "F.Cu") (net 9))
 (segment (start 74 67.25) (end 78.9 72.15) (width 0.6) (layer "F.Cu") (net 12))
 (segment (start 74 64.5) (end 74 67.25) (width 0.6) (layer "F.Cu") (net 12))
 (segment (start 107 83) (end 104 86) (width 0.6) (layer "F.Cu") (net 12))
 (segment (start 107.35 76) (end 107.35 80.15) (width 0.6) (layer "F.Cu") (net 12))
 (segment (start 100.65 72.15) (end 103 74.5) (width 0.6) (layer "F.Cu") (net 12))
 (segment (start 107 80.5) (end 107 83) (width 0.6) (layer "F.Cu") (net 12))
 (segment (start 107.35 80.15) (end 107 80.5) (width 0.6) (layer "F.Cu") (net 12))
 (segment (start 103 74.5) (end 105.85 74.5) (width 0.6) (layer "F.Cu") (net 12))
 (segment (start 78.9 72.15) (end 100.65 72.15) (width 0.6) (layer "F.Cu") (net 12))
 (segment (start 105.85 74.5) (end 107.35 76) (width 0.6) (layer "F.Cu") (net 12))
 (segment (start 71.5 74.5) (end 71.625 74.625) (width 0.6) (layer "F.Cu") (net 10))
 (segment (start 71.625 74.625) (end 81.2125 74.625) (width 0.6) (layer "F.Cu") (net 10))
 (segment (start 71 74.5) (end 71.5 74.5) (width 0.6) (layer "F.Cu") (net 10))
 (segment (start 71.5 89.9125) (end 72.2125 90.625) (width 0.6) (layer "F.Cu") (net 15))
 (segment (start 71.5 85) (end 71.5 89.9125) (width 0.6) (layer "F.Cu") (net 15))
 (segment (start 80 84.5) (end 87.392792 84.5) (width 0.6) (layer "F.Cu") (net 7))
 (segment (start 76.5 87.66) (end 76.84 87.66) (width 0.6) (layer "F.Cu") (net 7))
 (segment (start 74.5 91.1375) (end 74.5 89.66) (width 0.6) (layer "F.Cu") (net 7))
 (segment (start 87.392792 84.5) (end 88.635 85.742208) (width 0.6) (layer "F.Cu") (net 7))
 (segment (start 72.2125 93.425) (end 74.5 91.1375) (width 0.6) (layer "F.Cu") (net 7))
 (segment (start 76.84 87.66) (end 80 84.5) (width 0.6) (layer "F.Cu") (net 7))
 (segment (start 88.635 85.742208) (end 88.635 86.85) (width 0.6) (layer "F.Cu") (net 7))
 (segment (start 74.5 89.66) (end 76.5 87.66) (width 0.6) (layer "F.Cu") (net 7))
 (segment (start 76 64.5) (end 76 67.25) (width 0.6) (layer "F.Cu") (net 1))
 (segment (start 108.4 91.1) (end 108.4 74.55) (width 0.6) (layer "F.Cu") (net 1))
 (segment (start 76 67.25) (end 80 71.25) (width 0.6) (layer "F.Cu") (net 1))
 (segment (start 80 71.25) (end 105.1 71.25) (width 0.6) (layer "F.Cu") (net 1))
 (segment (start 105.1 71.25) (end 107.35 73.5) (width 0.6) (layer "F.Cu") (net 1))
 (segment (start 105 94.5) (end 108.4 91.1) (width 0.6) (layer "F.Cu") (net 1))
 (segment (start 108.4 74.55) (end 107.35 73.5) (width 0.6) (layer "F.Cu") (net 1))
 (segment (start 76.5 85.12) (end 78.02 83.6) (width 0.6) (layer "F.Cu") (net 6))
 (segment (start 88.6 83.6) (end 89.905 84.905) (width 0.6) (layer "F.Cu") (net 6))
 (segment (start 78.02 83.6) (end 88.6 83.6) (width 0.6) (layer "F.Cu") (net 6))
 (segment (start 89.905 84.905) (end 89.905 86.85) (width 0.6) (layer "F.Cu") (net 6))
 (segment (start 101 91) (end 104 88) (width 0.6) (layer "F.Cu") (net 4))
 (segment (start 86.555 91.89) (end 87.365 92.7) (width 0.6) (layer "F.Cu") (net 4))
 (segment (start 76.5 92.74) (end 77.35 91.89) (width 0.6) (layer "F.Cu") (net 4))
 (segment (start 87.365 92.7) (end 89.065 91) (width 0.6) (layer "F.Cu") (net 4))
 (segment (start 87.365 92.7) (end 87.365 94.15) (width 0.6) (layer "F.Cu") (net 4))
 (segment (start 89.065 91) (end 101 91) (width 0.6) (layer "F.Cu") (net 4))
 (segment (start 77.35 91.89) (end 86.555 91.89) (width 0.6) (layer "F.Cu") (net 4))
 (segment (start 87.365 85.745) (end 87.365 86.85) (width 0.6) (layer "F.Cu") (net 8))
 (segment (start 81.3 85.4) (end 87.02 85.4) (width 0.6) (layer "F.Cu") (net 8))
 (segment (start 76.5 90.2) (end 81.3 85.4) (width 0.6) (layer "F.Cu") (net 8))
 (segment (start 87.02 85.4) (end 87.365 85.745) (width 0.6) (layer "F.Cu") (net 8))
 (segment (start 82.425 97.82) (end 86.095 94.15) (width 0.6) (layer "F.Cu") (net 3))
 (segment (start 76.5 97.82) (end 82.425 97.82) (width 0.6) (layer "F.Cu") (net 3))
 (segment (start 75.05 100.96061) (end 75.89939 101.81) (width 0.6) (layer "F.Cu") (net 5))
 (segment (start 89.6 91.9) (end 88.635 92.865) (width 0.6) (layer "F.Cu") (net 5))
 (segment (start 82.08 101.81) (end 88.635 95.255) (width 0.6) (layer "F.Cu") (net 5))
 (segment (start 100.4 91.9) (end 89.6 91.9) (width 0.6) (layer "F.Cu") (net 5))
 (segment (start 88.635 92.865) (end 88.635 94.15) (width 0.6) (layer "F.Cu") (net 5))
 (segment (start 75.05 96.73) (end 75.05 100.96061) (width 0.6) (layer "F.Cu") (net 5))
 (segment (start 75.89939 101.81) (end 82.08 101.81) (width 0.6) (layer "F.Cu") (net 5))
 (segment (start 103 94.5) (end 100.4 91.9) (width 0.6) (layer "F.Cu") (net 5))
 (segment (start 88.635 95.255) (end 88.635 94.15) (width 0.6) (layer "F.Cu") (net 5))
 (segment (start 76.5 95.28) (end 75.05 96.73) (width 0.6) (layer "F.Cu") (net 5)))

